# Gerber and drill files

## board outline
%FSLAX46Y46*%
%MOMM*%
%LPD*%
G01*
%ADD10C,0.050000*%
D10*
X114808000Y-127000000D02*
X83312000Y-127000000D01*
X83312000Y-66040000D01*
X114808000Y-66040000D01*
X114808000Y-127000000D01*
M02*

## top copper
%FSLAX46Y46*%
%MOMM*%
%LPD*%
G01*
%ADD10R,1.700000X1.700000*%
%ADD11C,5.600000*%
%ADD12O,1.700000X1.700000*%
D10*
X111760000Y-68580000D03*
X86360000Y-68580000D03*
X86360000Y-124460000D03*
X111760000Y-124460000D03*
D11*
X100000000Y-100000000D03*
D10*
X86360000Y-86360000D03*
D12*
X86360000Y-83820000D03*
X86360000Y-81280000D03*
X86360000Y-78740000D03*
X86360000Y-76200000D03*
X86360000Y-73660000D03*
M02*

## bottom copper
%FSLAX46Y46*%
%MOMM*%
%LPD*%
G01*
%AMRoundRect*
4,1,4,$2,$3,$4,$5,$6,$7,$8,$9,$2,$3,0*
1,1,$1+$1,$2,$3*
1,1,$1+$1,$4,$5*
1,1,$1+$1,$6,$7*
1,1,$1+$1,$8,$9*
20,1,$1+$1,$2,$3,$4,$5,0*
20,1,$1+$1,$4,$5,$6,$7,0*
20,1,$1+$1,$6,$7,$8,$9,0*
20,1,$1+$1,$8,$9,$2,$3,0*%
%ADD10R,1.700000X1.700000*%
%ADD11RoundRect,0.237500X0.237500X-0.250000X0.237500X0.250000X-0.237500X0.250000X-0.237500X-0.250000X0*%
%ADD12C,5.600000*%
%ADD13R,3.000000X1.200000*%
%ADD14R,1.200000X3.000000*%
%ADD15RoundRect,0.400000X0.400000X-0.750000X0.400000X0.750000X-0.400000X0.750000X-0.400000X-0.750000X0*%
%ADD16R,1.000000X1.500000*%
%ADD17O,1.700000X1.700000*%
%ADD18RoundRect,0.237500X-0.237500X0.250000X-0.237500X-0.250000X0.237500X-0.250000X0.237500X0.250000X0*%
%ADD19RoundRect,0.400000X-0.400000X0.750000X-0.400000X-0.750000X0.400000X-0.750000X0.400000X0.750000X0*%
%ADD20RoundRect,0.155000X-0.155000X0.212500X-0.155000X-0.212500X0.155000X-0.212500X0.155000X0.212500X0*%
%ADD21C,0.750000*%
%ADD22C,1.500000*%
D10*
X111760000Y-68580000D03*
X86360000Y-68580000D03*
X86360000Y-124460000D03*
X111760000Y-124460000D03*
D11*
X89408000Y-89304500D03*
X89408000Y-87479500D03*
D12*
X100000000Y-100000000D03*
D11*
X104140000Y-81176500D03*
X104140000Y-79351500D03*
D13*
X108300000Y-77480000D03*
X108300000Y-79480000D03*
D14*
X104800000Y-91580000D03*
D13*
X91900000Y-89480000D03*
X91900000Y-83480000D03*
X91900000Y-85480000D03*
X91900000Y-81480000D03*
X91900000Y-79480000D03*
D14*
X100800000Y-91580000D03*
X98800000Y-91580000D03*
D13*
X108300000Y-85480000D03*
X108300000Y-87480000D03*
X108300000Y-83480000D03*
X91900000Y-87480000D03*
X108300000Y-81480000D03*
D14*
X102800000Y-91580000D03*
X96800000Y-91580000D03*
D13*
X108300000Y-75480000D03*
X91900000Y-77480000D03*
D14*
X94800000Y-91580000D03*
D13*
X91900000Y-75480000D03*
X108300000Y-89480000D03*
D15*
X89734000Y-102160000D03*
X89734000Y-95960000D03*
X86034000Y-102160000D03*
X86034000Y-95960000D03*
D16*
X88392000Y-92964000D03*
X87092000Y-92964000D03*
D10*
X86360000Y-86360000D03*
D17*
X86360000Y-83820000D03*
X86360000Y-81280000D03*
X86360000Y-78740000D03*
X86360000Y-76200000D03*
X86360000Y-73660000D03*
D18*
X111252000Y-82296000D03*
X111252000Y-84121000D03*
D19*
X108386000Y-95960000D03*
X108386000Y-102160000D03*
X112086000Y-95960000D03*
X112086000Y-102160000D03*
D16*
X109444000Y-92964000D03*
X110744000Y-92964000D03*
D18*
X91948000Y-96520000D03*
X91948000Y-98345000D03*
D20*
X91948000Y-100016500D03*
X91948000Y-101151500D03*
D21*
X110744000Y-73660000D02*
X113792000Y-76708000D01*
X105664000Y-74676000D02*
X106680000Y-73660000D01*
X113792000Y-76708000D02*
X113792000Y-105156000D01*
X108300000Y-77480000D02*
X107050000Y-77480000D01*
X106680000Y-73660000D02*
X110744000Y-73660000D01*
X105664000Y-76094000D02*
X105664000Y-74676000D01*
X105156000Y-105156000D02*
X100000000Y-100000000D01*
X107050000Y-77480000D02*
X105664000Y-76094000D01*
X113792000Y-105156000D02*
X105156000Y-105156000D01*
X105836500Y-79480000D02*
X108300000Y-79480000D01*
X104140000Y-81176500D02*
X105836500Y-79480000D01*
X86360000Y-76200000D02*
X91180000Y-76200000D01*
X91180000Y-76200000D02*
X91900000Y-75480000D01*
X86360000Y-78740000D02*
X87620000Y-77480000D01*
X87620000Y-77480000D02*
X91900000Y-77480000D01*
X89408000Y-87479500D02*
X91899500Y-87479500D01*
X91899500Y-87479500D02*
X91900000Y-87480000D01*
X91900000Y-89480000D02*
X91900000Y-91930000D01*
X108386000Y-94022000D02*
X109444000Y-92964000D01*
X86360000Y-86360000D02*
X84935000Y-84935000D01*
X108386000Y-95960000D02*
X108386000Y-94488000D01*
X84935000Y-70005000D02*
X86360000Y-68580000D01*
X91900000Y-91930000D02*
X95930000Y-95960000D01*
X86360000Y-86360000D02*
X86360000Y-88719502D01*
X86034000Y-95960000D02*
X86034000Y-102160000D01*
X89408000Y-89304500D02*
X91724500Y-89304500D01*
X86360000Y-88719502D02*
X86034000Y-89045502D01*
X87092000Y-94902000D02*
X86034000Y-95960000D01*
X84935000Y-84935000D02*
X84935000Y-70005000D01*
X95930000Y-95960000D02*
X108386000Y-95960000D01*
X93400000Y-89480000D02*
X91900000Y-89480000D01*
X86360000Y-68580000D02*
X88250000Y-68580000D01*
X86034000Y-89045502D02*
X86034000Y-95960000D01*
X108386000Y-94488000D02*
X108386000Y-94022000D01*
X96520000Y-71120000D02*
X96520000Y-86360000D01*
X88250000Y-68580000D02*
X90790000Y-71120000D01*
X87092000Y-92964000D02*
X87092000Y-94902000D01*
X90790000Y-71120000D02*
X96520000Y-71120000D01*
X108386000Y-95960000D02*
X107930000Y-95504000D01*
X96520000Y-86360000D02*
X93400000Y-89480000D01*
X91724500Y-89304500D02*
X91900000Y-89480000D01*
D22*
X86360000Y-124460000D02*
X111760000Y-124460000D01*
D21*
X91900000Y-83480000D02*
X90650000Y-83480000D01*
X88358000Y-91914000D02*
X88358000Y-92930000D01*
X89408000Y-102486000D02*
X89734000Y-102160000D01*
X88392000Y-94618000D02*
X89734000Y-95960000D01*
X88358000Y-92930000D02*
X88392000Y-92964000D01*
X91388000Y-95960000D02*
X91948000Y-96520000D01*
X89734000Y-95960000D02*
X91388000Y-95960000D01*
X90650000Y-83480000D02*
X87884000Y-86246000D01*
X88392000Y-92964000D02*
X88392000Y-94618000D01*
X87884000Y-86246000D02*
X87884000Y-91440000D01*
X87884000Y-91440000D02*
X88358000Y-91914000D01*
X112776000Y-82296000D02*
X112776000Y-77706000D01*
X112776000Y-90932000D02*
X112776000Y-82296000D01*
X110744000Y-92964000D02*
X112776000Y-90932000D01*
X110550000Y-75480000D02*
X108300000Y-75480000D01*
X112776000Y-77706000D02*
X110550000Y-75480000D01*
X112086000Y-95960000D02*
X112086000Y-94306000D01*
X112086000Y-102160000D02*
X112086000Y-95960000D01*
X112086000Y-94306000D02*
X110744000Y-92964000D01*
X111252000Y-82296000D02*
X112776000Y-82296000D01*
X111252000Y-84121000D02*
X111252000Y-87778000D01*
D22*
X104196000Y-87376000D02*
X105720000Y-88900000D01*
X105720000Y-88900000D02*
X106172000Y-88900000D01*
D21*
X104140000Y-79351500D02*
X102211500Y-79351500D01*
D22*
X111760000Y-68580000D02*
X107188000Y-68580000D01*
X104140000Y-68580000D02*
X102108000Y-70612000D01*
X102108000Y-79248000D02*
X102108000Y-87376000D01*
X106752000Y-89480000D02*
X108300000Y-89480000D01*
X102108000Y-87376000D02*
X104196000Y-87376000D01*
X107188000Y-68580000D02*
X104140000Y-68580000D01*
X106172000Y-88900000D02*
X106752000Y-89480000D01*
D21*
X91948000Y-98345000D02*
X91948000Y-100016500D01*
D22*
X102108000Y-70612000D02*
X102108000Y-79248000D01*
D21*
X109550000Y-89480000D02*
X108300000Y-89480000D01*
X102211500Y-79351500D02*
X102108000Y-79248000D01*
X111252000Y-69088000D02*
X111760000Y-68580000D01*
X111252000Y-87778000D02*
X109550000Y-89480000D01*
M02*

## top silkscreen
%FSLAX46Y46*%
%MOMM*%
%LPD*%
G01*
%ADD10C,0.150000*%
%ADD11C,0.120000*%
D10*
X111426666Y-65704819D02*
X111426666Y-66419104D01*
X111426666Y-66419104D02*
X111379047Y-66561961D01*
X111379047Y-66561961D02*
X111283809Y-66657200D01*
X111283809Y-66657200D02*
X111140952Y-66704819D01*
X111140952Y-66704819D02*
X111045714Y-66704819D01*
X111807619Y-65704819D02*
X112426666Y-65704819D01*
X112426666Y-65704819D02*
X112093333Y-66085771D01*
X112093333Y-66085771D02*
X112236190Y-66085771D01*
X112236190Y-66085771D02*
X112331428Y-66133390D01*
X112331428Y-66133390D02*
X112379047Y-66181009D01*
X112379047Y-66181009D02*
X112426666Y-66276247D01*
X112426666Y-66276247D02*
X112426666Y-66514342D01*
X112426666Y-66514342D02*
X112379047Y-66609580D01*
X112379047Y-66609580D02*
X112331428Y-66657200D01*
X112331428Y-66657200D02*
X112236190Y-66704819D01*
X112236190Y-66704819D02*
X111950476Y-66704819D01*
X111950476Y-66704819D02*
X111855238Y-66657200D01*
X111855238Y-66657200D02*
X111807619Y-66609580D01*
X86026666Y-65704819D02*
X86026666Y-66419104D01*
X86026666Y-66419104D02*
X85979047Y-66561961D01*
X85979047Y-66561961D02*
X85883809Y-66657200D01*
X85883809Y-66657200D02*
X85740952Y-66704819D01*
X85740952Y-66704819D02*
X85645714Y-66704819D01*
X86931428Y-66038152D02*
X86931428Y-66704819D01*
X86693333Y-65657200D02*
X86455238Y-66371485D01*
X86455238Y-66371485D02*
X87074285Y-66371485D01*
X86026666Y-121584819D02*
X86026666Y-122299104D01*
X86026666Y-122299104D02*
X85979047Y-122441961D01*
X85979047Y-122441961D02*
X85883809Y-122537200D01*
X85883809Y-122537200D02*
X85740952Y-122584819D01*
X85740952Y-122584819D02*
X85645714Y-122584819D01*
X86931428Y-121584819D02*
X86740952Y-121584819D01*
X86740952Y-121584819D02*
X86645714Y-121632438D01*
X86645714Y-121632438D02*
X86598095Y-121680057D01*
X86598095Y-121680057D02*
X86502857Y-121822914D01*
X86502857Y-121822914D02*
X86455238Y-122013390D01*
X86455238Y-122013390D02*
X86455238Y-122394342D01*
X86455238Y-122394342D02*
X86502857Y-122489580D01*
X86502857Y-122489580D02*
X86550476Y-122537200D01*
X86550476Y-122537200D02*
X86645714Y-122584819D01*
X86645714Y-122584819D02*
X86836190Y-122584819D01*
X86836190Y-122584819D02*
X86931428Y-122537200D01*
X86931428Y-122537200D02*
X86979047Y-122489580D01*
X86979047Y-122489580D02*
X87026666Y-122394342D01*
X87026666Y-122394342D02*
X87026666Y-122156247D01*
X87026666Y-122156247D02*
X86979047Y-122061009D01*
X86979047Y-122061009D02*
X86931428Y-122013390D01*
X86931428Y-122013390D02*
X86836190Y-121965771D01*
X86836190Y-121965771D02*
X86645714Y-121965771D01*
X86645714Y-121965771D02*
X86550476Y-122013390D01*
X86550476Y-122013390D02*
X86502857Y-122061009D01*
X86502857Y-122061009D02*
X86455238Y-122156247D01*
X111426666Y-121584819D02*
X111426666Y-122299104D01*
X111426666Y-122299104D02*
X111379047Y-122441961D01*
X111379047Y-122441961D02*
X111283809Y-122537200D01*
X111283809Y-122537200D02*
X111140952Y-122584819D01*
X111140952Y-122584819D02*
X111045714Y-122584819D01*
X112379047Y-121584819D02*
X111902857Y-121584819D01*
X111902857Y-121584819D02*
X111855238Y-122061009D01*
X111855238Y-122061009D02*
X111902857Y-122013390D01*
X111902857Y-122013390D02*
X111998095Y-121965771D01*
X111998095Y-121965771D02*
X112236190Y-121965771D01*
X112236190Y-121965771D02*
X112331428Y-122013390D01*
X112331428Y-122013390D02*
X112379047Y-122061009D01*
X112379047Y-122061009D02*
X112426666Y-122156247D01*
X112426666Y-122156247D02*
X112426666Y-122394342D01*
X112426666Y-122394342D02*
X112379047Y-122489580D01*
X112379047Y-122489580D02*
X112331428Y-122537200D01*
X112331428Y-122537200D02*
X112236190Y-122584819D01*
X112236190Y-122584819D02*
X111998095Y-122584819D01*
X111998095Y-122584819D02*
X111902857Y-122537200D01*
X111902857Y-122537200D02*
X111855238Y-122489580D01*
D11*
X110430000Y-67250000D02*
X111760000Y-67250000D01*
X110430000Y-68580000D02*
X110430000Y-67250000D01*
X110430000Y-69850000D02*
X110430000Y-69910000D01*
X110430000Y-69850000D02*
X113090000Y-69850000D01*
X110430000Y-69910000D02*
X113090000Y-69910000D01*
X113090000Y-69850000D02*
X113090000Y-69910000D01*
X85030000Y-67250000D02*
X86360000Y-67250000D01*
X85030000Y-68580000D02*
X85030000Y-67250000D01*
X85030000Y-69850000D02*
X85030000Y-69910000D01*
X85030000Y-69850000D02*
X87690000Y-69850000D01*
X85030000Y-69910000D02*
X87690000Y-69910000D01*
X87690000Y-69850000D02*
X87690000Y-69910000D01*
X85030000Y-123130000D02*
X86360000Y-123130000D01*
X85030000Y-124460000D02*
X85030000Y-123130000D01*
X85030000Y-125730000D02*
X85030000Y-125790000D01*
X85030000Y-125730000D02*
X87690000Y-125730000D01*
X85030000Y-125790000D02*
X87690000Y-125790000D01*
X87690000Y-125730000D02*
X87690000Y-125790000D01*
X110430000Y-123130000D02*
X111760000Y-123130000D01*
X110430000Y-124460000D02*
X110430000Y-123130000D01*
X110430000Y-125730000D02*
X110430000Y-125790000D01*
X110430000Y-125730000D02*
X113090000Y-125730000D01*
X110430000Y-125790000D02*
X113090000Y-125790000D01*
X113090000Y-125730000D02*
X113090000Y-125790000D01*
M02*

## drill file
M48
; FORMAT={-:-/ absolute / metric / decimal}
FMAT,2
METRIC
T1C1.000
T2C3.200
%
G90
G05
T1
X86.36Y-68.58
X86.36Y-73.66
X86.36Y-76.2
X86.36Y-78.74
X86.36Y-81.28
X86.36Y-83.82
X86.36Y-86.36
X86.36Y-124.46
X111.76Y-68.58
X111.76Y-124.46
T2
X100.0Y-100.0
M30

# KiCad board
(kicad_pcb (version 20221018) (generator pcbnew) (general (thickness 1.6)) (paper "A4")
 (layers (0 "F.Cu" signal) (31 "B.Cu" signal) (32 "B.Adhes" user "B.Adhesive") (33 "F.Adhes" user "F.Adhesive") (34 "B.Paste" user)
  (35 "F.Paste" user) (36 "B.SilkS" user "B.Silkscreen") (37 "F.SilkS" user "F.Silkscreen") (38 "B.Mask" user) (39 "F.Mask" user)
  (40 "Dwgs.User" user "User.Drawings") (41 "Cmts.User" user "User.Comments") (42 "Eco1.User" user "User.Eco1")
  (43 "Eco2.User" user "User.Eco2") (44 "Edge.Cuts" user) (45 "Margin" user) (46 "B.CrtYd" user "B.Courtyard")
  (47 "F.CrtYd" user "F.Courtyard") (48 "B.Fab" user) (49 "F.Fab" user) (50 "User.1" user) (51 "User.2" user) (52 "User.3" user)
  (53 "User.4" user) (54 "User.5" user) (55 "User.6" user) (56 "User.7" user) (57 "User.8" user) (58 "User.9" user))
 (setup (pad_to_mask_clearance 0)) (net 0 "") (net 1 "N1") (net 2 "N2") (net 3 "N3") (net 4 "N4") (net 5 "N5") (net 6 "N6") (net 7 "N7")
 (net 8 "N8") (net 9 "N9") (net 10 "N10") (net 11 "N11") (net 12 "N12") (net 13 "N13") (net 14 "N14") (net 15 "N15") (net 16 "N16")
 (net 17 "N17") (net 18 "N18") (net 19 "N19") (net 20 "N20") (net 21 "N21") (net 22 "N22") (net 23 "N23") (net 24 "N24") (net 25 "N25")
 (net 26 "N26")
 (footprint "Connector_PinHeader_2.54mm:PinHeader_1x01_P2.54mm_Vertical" (layer "F.Cu") (at 111.76 68.58)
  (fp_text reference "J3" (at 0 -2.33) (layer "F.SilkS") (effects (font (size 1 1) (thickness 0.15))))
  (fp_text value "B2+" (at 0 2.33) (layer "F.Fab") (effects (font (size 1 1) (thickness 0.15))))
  (fp_line (start -1.33 -1.33) (end 0 -1.33) (stroke (width 0.12) (type solid)) (layer "F.SilkS"))
  (fp_line (start -1.33 0) (end -1.33 -1.33) (stroke (width 0.12) (type solid)) (layer "F.SilkS"))
  (fp_line (start -1.33 1.27) (end -1.33 1.33) (stroke (width 0.12) (type solid)) (layer "F.SilkS"))
  (fp_line (start -1.33 1.27) (end 1.33 1.27) (stroke (width 0.12) (type solid)) (layer "F.SilkS"))
  (fp_line (start -1.33 1.33) (end 1.33 1.33) (stroke (width 0.12) (type solid)) (layer "F.SilkS"))
  (fp_line (start 1.33 1.27) (end 1.33 1.33) (stroke (width 0.12) (type solid)) (layer "F.SilkS"))
  (pad "1" thru_hole rect (at 0 0) (size 1.7 1.7) (drill 1) (layers "*.Cu" "*.Mask") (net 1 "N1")))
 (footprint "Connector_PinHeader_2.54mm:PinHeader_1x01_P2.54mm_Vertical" (layer "F.Cu") (at 86.36 68.58)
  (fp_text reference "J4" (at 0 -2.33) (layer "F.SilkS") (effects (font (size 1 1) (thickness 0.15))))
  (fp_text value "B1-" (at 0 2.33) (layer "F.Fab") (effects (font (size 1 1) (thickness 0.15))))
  (fp_line (start -1.33 -1.33) (end 0 -1.33) (stroke (width 0.12) (type solid)) (layer "F.SilkS"))
  (fp_line (start -1.33 0) (end -1.33 -1.33) (stroke (width 0.12) (type solid)) (layer "F.SilkS"))
  (fp_line (start -1.33 1.27) (end -1.33 1.33) (stroke (width 0.12) (type solid)) (layer "F.SilkS"))
  (fp_line (start -1.33 1.27) (end 1.33 1.27) (stroke (width 0.12) (type solid)) (layer "F.SilkS"))
  (fp_line (start -1.33 1.33) (end 1.33 1.33) (stroke (width 0.12) (type solid)) (layer "F.SilkS"))
  (fp_line (start 1.33 1.27) (end 1.33 1.33) (stroke (width 0.12) (type solid)) (layer "F.SilkS"))
  (pad "1" thru_hole rect (at 0 0) (size 1.7 1.7) (drill 1) (layers "*.Cu" "*.Mask") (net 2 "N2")))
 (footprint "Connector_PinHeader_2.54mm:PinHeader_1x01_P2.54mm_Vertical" (layer "F.Cu") (at 86.36 124.46)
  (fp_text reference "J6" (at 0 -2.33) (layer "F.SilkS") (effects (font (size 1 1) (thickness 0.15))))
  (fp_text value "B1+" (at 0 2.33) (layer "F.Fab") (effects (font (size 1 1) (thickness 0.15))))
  (fp_line (start -1.33 -1.33) (end 0 -1.33) (stroke (width 0.12) (type solid)) (layer "F.SilkS"))
  (fp_line (start -1.33 0) (end -1.33 -1.33) (stroke (width 0.12) (type solid)) (layer "F.SilkS"))
  (fp_line (start -1.33 1.27) (end -1.33 1.33) (stroke (width 0.12) (type solid)) (layer "F.SilkS"))
  (fp_line (start -1.33 1.27) (end 1.33 1.27) (stroke (width 0.12) (type solid)) (layer "F.SilkS"))
  (fp_line (start -1.33 1.33) (end 1.33 1.33) (stroke (width 0.12) (type solid)) (layer "F.SilkS"))
  (fp_line (start 1.33 1.27) (end 1.33 1.33) (stroke (width 0.12) (type solid)) (layer "F.SilkS"))
  (pad "1" thru_hole rect (at 0 0) (size 1.7 1.7) (drill 1) (layers "*.Cu" "*.Mask") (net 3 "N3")))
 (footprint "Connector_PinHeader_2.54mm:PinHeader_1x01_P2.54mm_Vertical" (layer "F.Cu") (at 111.76 124.46)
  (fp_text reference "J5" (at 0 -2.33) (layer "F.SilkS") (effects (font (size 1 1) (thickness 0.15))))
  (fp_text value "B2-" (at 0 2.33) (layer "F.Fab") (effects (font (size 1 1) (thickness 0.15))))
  (fp_line (start -1.33 -1.33) (end 0 -1.33) (stroke (width 0.12) (type solid)) (layer "F.SilkS"))
  (fp_line (start -1.33 0) (end -1.33 -1.33) (stroke (width 0.12) (type solid)) (layer "F.SilkS"))
  (fp_line (start -1.33 1.27) (end -1.33 1.33) (stroke (width 0.12) (type solid)) (layer "F.SilkS"))
  (fp_line (start -1.33 1.27) (end 1.33 1.27) (stroke (width 0.12) (type solid)) (layer "F.SilkS"))
  (fp_line (start -1.33 1.33) (end 1.33 1.33) (stroke (width 0.12) (type solid)) (layer "F.SilkS"))
  (fp_line (start 1.33 1.27) (end 1.33 1.33) (stroke (width 0.12) (type solid)) (layer "F.SilkS"))
  (pad "1" thru_hole rect (at 0 0) (size 1.7 1.7) (drill 1) (layers "*.Cu" "*.Mask") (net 3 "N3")))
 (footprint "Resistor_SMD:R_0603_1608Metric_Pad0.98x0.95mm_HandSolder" (layer "B.Cu") (at 89.408 88.392 90)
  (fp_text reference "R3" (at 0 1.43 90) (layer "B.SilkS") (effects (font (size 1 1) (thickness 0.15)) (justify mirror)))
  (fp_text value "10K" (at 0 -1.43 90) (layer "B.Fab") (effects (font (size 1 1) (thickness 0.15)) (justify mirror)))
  (pad "1" smd roundrect (at -0.9125 0 90) (size 0.975 0.95) (layers "B.Cu" "B.Paste" "B.Mask") (roundrect_rratio 0.25) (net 2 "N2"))
  (pad "2" smd roundrect (at 0.9125 0 90) (size 0.975 0.95) (layers "B.Cu" "B.Paste" "B.Mask") (roundrect_rratio 0.25) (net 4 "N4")))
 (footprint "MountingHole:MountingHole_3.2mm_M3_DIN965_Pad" (layer "B.Cu") (at 100 100 180)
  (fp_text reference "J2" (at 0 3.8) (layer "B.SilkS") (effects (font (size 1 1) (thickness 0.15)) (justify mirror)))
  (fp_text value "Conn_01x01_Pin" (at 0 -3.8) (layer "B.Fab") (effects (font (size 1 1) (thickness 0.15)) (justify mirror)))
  (pad "1" thru_hole circle (at 0 0 180) (size 5.6 5.6) (drill 3.2) (layers "*.Cu" "*.Mask") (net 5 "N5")))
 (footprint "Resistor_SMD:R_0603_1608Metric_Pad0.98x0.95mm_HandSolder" (layer "B.Cu") (at 104.14 80.264 90)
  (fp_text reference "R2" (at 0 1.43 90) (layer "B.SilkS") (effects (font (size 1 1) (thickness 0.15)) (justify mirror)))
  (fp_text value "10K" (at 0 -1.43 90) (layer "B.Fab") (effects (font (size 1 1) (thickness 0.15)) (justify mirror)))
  (pad "1" smd roundrect (at -0.9125 0 90) (size 0.975 0.95) (layers "B.Cu" "B.Paste" "B.Mask") (roundrect_rratio 0.25) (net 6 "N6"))
  (pad "2" smd roundrect (at 0.9125 0 90) (size 0.975 0.95) (layers "B.Cu" "B.Paste" "B.Mask") (roundrect_rratio 0.25) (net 1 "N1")))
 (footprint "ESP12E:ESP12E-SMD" (layer "B.Cu") (at 100 81.28 180)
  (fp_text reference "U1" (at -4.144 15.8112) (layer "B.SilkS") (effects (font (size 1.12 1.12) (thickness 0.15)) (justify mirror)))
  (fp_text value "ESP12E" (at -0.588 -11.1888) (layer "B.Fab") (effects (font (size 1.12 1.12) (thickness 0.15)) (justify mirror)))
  (pad "ADC" smd rect (at -8.3 3.8 180) (size 3 1.2) (layers "B.Cu" "B.Paste" "B.Mask") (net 5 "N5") (solder_mask_margin 0.102))
  (pad "CH_PD" smd rect (at -8.3 1.8 180) (size 3 1.2) (layers "B.Cu" "B.Paste" "B.Mask") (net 6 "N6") (solder_mask_margin 0.102))
  (pad "CS0" smd rect (at -4.8 -10.3 90) (size 3 1.2) (layers "B.Cu" "B.Paste" "B.Mask") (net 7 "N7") (solder_mask_margin 0.102))
  (pad "GND" smd rect (at 8.1 -8.2 180) (size 3 1.2) (layers "B.Cu" "B.Paste" "B.Mask") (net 2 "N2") (solder_mask_margin 0.102))
  (pad "GPIO0" smd rect (at 8.1 -2.2 180) (size 3 1.2) (layers "B.Cu" "B.Paste" "B.Mask") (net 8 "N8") (solder_mask_margin 0.102))
  (pad "GPIO2" smd rect (at 8.1 -4.2 180) (size 3 1.2) (layers "B.Cu" "B.Paste" "B.Mask") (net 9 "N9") (solder_mask_margin 0.102))
  (pad "GPIO4" smd rect (at 8.1 -0.2 180) (size 3 1.2) (layers "B.Cu" "B.Paste" "B.Mask") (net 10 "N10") (solder_mask_margin 0.102))
  (pad "GPIO5" smd rect (at 8.1 1.8 180) (size 3 1.2) (layers "B.Cu" "B.Paste" "B.Mask") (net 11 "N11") (solder_mask_margin 0.102))
  (pad "GPIO9" smd rect (at -0.8 -10.3 90) (size 3 1.2) (layers "B.Cu" "B.Paste" "B.Mask") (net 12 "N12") (solder_mask_margin 0.102))
  (pad "GPIO10" smd rect (at 1.2 -10.3 90) (size 3 1.2) (layers "B.Cu" "B.Paste" "B.Mask") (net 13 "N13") (solder_mask_margin 0.102))
  (pad "GPIO12" smd rect (at -8.3 -4.2 180) (size 3 1.2) (layers "B.Cu" "B.Paste" "B.Mask") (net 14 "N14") (solder_mask_margin 0.102))
  (pad "GPIO13" smd rect (at -8.3 -6.2 180) (size 3 1.2) (layers "B.Cu" "B.Paste" "B.Mask") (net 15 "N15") (solder_mask_margin 0.102))
  (pad "GPIO14" smd rect (at -8.3 -2.2 180) (size 3 1.2) (layers "B.Cu" "B.Paste" "B.Mask") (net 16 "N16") (solder_mask_margin 0.102))
  (pad "GPIO15" smd rect (at 8.1 -6.2 180) (size 3 1.2) (layers "B.Cu" "B.Paste" "B.Mask") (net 4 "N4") (solder_mask_margin 0.102))
  (pad "GPIO16" smd rect (at -8.3 -0.2 180) (size 3 1.2) (layers "B.Cu" "B.Paste" "B.Mask") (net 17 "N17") (solder_mask_margin 0.102))
  (pad "MISO" smd rect (at -2.8 -10.3 90) (size 3 1.2) (layers "B.Cu" "B.Paste" "B.Mask") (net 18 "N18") (solder_mask_margin 0.102))
  (pad "MOSI" smd rect (at 3.2 -10.3 90) (size 3 1.2) (layers "B.Cu" "B.Paste" "B.Mask") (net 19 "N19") (solder_mask_margin 0.102))
  (pad "RESET" smd rect (at -8.3 5.8 180) (size 3 1.2) (layers "B.Cu" "B.Paste" "B.Mask") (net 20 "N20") (solder_mask_margin 0.102))
  (pad "RXD0" smd rect (at 8.1 3.8 180) (size 3 1.2) (layers "B.Cu" "B.Paste" "B.Mask") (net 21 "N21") (solder_mask_margin 0.102))
  (pad "SCLK" smd rect (at 5.2 -10.3 90) (size 3 1.2) (layers "B.Cu" "B.Paste" "B.Mask") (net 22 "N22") (solder_mask_margin 0.102))
  (pad "TXD0" smd rect (at 8.1 5.8 180) (size 3 1.2) (layers "B.Cu" "B.Paste" "B.Mask") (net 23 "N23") (solder_mask_margin 0.102))
  (pad "VCC" smd rect (at -8.3 -8.2 180) (size 3 1.2) (layers "B.Cu" "B.Paste" "B.Mask") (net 1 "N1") (solder_mask_margin 0.102)))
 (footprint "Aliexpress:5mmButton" (layer "B.Cu") (at 87.884 99.06 90)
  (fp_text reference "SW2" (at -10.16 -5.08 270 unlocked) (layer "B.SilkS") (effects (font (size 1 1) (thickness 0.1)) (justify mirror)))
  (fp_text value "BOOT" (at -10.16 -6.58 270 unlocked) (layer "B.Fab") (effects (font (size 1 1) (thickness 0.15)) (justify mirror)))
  (pad "1" smd roundrect (at -3.1 1.85 90) (size 2.3 1.6) (layers "B.Cu" "B.Paste" "B.Mask") (roundrect_rratio 0.25) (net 8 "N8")
   (thermal_bridge_angle 45))
  (pad "1" smd roundrect (at 3.1 1.85 90) (size 2.3 1.6) (layers "B.Cu" "B.Paste" "B.Mask") (roundrect_rratio 0.25) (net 8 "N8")
   (thermal_bridge_angle 45))
  (pad "2" smd roundrect (at -3.1 -1.85 90) (size 2.3 1.6) (layers "B.Cu" "B.Paste" "B.Mask") (roundrect_rratio 0.25) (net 2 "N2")
   (thermal_bridge_angle 45))
  (pad "2" smd roundrect (at 3.1 -1.85 90) (size 2.3 1.6) (layers "B.Cu" "B.Paste" "B.Mask") (roundrect_rratio 0.25) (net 2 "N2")
   (thermal_bridge_angle 45)))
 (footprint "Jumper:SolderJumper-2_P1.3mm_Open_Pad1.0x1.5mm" (layer "B.Cu") (at 87.742 92.964 180) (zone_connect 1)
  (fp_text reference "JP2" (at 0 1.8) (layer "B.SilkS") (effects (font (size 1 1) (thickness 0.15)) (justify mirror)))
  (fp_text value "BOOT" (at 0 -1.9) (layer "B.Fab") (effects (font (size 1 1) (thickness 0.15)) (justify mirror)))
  (pad "1" smd rect (at -0.65 0 180) (size 1 1.5) (layers "B.Cu" "B.Mask") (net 8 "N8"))
  (pad "2" smd rect (at 0.65 0 180) (size 1 1.5) (layers "B.Cu" "B.Mask") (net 2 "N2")))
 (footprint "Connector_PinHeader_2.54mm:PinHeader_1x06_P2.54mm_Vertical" (layer "B.Cu") (at 86.36 86.36)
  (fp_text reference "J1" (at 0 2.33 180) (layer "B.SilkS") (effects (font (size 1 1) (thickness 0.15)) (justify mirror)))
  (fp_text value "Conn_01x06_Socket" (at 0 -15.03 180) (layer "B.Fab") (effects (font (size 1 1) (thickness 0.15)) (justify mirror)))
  (pad "1" thru_hole rect (at 0 0) (size 1.7 1.7) (drill 1) (layers "*.Cu" "*.Mask") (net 2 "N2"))
  (pad "2" thru_hole oval (at 0 -2.54) (size 1.7 1.7) (drill 1) (layers "*.Cu" "*.Mask") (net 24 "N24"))
  (pad "3" thru_hole oval (at 0 -5.08) (size 1.7 1.7) (drill 1) (layers "*.Cu" "*.Mask") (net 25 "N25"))
  (pad "4" thru_hole oval (at 0 -7.62) (size 1.7 1.7) (drill 1) (layers "*.Cu" "*.Mask") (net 21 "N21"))
  (pad "5" thru_hole oval (at 0 -10.16) (size 1.7 1.7) (drill 1) (layers "*.Cu" "*.Mask") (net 23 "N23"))
  (pad "6" thru_hole oval (at 0 -12.7) (size 1.7 1.7) (drill 1) (layers "*.Cu" "*.Mask") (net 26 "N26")))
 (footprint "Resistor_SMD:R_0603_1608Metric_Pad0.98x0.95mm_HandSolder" (layer "B.Cu") (at 111.252 83.2085 -90)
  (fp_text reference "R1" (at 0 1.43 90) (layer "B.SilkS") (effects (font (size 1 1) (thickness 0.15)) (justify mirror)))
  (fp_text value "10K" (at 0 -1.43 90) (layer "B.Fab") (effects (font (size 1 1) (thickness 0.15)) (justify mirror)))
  (pad "1" smd roundrect (at -0.9125 0 270) (size 0.975 0.95) (layers "B.Cu" "B.Paste" "B.Mask") (roundrect_rratio 0.25) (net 20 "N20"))
  (pad "2" smd roundrect (at 0.9125 0 270) (size 0.975 0.95) (layers "B.Cu" "B.Paste" "B.Mask") (roundrect_rratio 0.25) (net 1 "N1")))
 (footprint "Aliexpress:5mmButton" (layer "B.Cu") (at 110.236 99.06 -90)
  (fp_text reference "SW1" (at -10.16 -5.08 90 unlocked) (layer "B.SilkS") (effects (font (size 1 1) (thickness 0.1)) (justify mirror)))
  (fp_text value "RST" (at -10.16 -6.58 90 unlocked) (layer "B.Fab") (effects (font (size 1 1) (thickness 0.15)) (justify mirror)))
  (pad "1" smd roundrect (at -3.1 1.85 270) (size 2.3 1.6) (layers "B.Cu" "B.Paste" "B.Mask") (roundrect_rratio 0.25) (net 2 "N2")
   (thermal_bridge_angle 45))
  (pad "1" smd roundrect (at 3.1 1.85 270) (size 2.3 1.6) (layers "B.Cu" "B.Paste" "B.Mask") (roundrect_rratio 0.25) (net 2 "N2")
   (thermal_bridge_angle 45))
  (pad "2" smd roundrect (at -3.1 -1.85 270) (size 2.3 1.6) (layers "B.Cu" "B.Paste" "B.Mask") (roundrect_rratio 0.25) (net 20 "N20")
   (thermal_bridge_angle 45))
  (pad "2" smd roundrect (at 3.1 -1.85 270) (size 2.3 1.6) (layers "B.Cu" "B.Paste" "B.Mask") (roundrect_rratio 0.25) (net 20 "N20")
   (thermal_bridge_angle 45)))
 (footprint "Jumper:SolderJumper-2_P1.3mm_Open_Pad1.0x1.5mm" (layer "B.Cu") (at 110.094 92.964) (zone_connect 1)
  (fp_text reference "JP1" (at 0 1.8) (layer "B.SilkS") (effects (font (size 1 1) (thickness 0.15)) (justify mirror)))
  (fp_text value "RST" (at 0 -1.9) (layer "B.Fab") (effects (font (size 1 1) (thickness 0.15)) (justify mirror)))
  (pad "1" smd rect (at -0.65 0) (size 1 1.5) (layers "B.Cu" "B.Mask") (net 2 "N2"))
  (pad "2" smd rect (at 0.65 0) (size 1 1.5) (layers "B.Cu" "B.Mask") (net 20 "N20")))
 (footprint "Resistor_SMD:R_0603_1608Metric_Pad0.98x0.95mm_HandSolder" (layer "B.Cu") (at 91.948 97.4325 -90)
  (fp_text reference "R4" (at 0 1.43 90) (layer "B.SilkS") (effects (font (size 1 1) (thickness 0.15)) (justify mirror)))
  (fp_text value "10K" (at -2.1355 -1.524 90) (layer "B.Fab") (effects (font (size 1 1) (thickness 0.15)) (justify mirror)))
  (pad "1" smd roundrect (at -0.9125 0 270) (size 0.975 0.95) (layers "B.Cu" "B.Paste" "B.Mask") (roundrect_rratio 0.25) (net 8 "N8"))
  (pad "2" smd roundrect (at 0.9125 0 270) (size 0.975 0.95) (layers "B.Cu" "B.Paste" "B.Mask") (roundrect_rratio 0.25) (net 1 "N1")))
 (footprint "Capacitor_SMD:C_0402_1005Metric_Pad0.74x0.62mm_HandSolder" (layer "B.Cu") (at 91.948 100.584 -90)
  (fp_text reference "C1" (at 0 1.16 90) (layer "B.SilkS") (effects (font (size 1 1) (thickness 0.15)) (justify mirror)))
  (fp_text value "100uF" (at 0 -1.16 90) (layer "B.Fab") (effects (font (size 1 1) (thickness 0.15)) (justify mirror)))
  (pad "1" smd roundrect (at -0.5675 0 270) (size 0.735 0.62) (layers "B.Cu" "B.Paste" "B.Mask") (roundrect_rratio 0.25) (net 1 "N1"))
  (pad "2" smd roundrect (at 0.5675 0 270) (size 0.735 0.62) (layers "B.Cu" "B.Paste" "B.Mask") (roundrect_rratio 0.25) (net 2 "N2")))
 (gr_poly
  (pts (xy 114.808 127) (xy 83.312 127) (xy 83.312 66.04) (xy 114.808 66.04)) (stroke (width 0.05) (type solid)) (fill none)
  (layer "Edge.Cuts"))
 (segment (start 110.744 73.66) (end 113.792 76.708) (width 0.75) (layer "B.Cu") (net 5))
 (segment (start 105.664 74.676) (end 106.68 73.66) (width 0.75) (layer "B.Cu") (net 5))
 (segment (start 113.792 76.708) (end 113.792 105.156) (width 0.75) (layer "B.Cu") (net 5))
 (segment (start 108.3 77.48) (end 107.05 77.48) (width 0.75) (layer "B.Cu") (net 5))
 (segment (start 106.68 73.66) (end 110.744 73.66) (width 0.75) (layer "B.Cu") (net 5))
 (segment (start 105.664 76.094) (end 105.664 74.676) (width 0.75) (layer "B.Cu") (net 5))
 (segment (start 105.156 105.156) (end 100 100) (width 0.75) (layer "B.Cu") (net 5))
 (segment (start 107.05 77.48) (end 105.664 76.094) (width 0.75) (layer "B.Cu") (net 5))
 (segment (start 113.792 105.156) (end 105.156 105.156) (width 0.75) (layer "B.Cu") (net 5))
 (segment (start 105.8365 79.48) (end 108.3 79.48) (width 0.75) (layer "B.Cu") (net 6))
 (segment (start 104.14 81.1765) (end 105.8365 79.48) (width 0.75) (layer "B.Cu") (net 6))
 (segment (start 86.36 76.2) (end 91.18 76.2) (width 0.75) (layer "B.Cu") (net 23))
 (segment (start 91.18 76.2) (end 91.9 75.48) (width 0.75) (layer "B.Cu") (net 23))
 (segment (start 86.36 78.74) (end 87.62 77.48) (width 0.75) (layer "B.Cu") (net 21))
 (segment (start 87.62 77.48) (end 91.9 77.48) (width 0.75) (layer "B.Cu") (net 21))
 (segment (start 89.408 87.4795) (end 91.8995 87.4795) (width 0.75) (layer "B.Cu") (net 4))
 (segment (start 91.8995 87.4795) (end 91.9 87.48) (width 0.75) (layer "B.Cu") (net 4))
 (segment (start 91.9 89.48) (end 91.9 91.93) (width 0.75) (layer "B.Cu") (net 2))
 (segment (start 108.386 94.022) (end 109.444 92.964) (width 0.75) (layer "B.Cu") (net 2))
 (segment (start 86.36 86.36) (end 84.935 84.935) (width 0.75) (layer "B.Cu") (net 2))
 (segment (start 108.386 95.96) (end 108.386 94.488) (width 0.75) (layer "B.Cu") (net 2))
 (segment (start 84.935 70.005) (end 86.36 68.58) (width 0.75) (layer "B.Cu") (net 2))
 (segment (start 91.9 91.93) (end 95.93 95.96) (width 0.75) (layer "B.Cu") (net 2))
 (segment (start 86.36 86.36) (end 86.36 88.719502) (width 0.75) (layer "B.Cu") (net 2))
 (segment (start 86.034 95.96) (end 86.034 102.16) (width 0.75) (layer "B.Cu") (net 2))
 (segment (start 89.408 89.3045) (end 91.7245 89.3045) (width 0.75) (layer "B.Cu") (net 2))
 (segment (start 86.36 88.719502) (end 86.034 89.045502) (width 0.75) (layer "B.Cu") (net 2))
 (segment (start 87.092 94.902) (end 86.034 95.96) (width 0.75) (layer "B.Cu") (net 2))
 (segment (start 84.935 84.935) (end 84.935 70.005) (width 0.75) (layer "B.Cu") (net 2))
 (segment (start 95.93 95.96) (end 108.386 95.96) (width 0.75) (layer "B.Cu") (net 2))
 (segment (start 93.4 89.48) (end 91.9 89.48) (width 0.75) (layer "B.Cu") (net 2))
 (segment (start 86.36 68.58) (end 88.25 68.58) (width 0.75) (layer "B.Cu") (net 2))
 (segment (start 86.034 89.045502) (end 86.034 95.96) (width 0.75) (layer "B.Cu") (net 2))
 (segment (start 108.386 94.488) (end 108.386 94.022) (width 0.75) (layer "B.Cu") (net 2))
 (segment (start 96.52 71.12) (end 96.52 86.36) (width 0.75) (layer "B.Cu") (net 2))
 (segment (start 88.25 68.58) (end 90.79 71.12) (width 0.75) (layer "B.Cu") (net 2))
 (segment (start 87.092 92.964) (end 87.092 94.902) (width 0.75) (layer "B.Cu") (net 2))
 (segment (start 90.79 71.12) (end 96.52 71.12) (width 0.75) (layer "B.Cu") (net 2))
 (segment (start 108.386 95.96) (end 107.93 95.504) (width 0.75) (layer "B.Cu") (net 2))
 (segment (start 96.52 86.36) (end 93.4 89.48) (width 0.75) (layer "B.Cu") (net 2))
 (segment (start 91.7245 89.3045) (end 91.9 89.48) (width 0.75) (layer "B.Cu") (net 2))
 (segment (start 86.36 124.46) (end 111.76 124.46) (width 1.5) (layer "B.Cu") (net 3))
 (segment (start 91.9 83.48) (end 90.65 83.48) (width 0.75) (layer "B.Cu") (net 8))
 (segment (start 88.358 91.914) (end 88.358 92.93) (width 0.75) (layer "B.Cu") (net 8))
 (segment (start 89.408 102.486) (end 89.734 102.16) (width 0.75) (layer "B.Cu") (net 8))
 (segment (start 88.392 94.618) (end 89.734 95.96) (width 0.75) (layer "B.Cu") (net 8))
 (segment (start 88.358 92.93) (end 88.392 92.964) (width 0.75) (layer "B.Cu") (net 8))
 (segment (start 91.388 95.96) (end 91.948 96.52) (width 0.75) (layer "B.Cu") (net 8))
 (segment (start 89.734 95.96) (end 91.388 95.96) (width 0.75) (layer "B.Cu") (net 8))
 (segment (start 90.65 83.48) (end 87.884 86.246) (width 0.75) (layer "B.Cu") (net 8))
 (segment (start 88.392 92.964) (end 88.392 94.618) (width 0.75) (layer "B.Cu") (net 8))
 (segment (start 87.884 86.246) (end 87.884 91.44) (width 0.75) (layer "B.Cu") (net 8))
 (segment (start 87.884 91.44) (end 88.358 91.914) (width 0.75) (layer "B.Cu") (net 8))
 (segment (start 112.776 82.296) (end 112.776 77.706) (width 0.75) (layer "B.Cu") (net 20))
 (segment (start 112.776 90.932) (end 112.776 82.296) (width 0.75) (layer "B.Cu") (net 20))
 (segment (start 110.744 92.964) (end 112.776 90.932) (width 0.75) (layer "B.Cu") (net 20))
 (segment (start 110.55 75.48) (end 108.3 75.48) (width 0.75) (layer "B.Cu") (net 20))
 (segment (start 112.776 77.706) (end 110.55 75.48) (width 0.75) (layer "B.Cu") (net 20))
 (segment (start 112.086 95.96) (end 112.086 94.306) (width 0.75) (layer "B.Cu") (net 20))
 (segment (start 112.086 102.16) (end 112.086 95.96) (width 0.75) (layer "B.Cu") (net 20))
 (segment (start 112.086 94.306) (end 110.744 92.964) (width 0.75) (layer "B.Cu") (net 20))
 (segment (start 111.252 82.296) (end 112.776 82.296) (width 0.75) (layer "B.Cu") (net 20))
 (segment (start 111.252 84.121) (end 111.252 87.778) (width 0.75) (layer "B.Cu") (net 1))
 (segment (start 104.196 87.376) (end 105.72 88.9) (width 1.5) (layer "B.Cu") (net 1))
 (segment (start 105.72 88.9) (end 106.172 88.9) (width 1.5) (layer "B.Cu") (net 1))
 (segment (start 104.14 79.3515) (end 102.2115 79.3515) (width 0.75) (layer "B.Cu") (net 1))
 (segment (start 111.76 68.58) (end 107.188 68.58) (width 1.5) (layer "B.Cu") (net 1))
 (segment (start 104.14 68.58) (end 102.108 70.612) (width 1.5) (layer "B.Cu") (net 1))
 (segment (start 102.108 79.248) (end 102.108 87.376) (width 1.5) (layer "B.Cu") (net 1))
 (segment (start 106.752 89.48) (end 108.3 89.48) (width 1.5) (layer "B.Cu") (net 1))
 (segment (start 102.108 87.376) (end 104.196 87.376) (width 1.5) (layer "B.Cu") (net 1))
 (segment (start 107.188 68.58) (end 104.14 68.58) (width 1.5) (layer "B.Cu") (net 1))
 (segment (start 106.172 88.9) (end 106.752 89.48) (width 1.5) (layer "B.Cu") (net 1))
 (segment (start 91.948 98.345) (end 91.948 100.0165) (width 0.75) (layer "B.Cu") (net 1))
 (segment (start 102.108 70.612) (end 102.108 79.248) (width 1.5) (layer "B.Cu") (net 1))
 (segment (start 109.55 89.48) (end 108.3 89.48) (width 0.75) (layer "B.Cu") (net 1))
 (segment (start 102.2115 79.3515) (end 102.108 79.248) (width 0.75) (layer "B.Cu") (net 1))
 (segment (start 111.252 69.088) (end 111.76 68.58) (width 0.75) (layer "B.Cu") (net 1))
 (segment (start 111.252 87.778) (end 109.55 89.48) (width 0.75) (layer "B.Cu") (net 1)))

